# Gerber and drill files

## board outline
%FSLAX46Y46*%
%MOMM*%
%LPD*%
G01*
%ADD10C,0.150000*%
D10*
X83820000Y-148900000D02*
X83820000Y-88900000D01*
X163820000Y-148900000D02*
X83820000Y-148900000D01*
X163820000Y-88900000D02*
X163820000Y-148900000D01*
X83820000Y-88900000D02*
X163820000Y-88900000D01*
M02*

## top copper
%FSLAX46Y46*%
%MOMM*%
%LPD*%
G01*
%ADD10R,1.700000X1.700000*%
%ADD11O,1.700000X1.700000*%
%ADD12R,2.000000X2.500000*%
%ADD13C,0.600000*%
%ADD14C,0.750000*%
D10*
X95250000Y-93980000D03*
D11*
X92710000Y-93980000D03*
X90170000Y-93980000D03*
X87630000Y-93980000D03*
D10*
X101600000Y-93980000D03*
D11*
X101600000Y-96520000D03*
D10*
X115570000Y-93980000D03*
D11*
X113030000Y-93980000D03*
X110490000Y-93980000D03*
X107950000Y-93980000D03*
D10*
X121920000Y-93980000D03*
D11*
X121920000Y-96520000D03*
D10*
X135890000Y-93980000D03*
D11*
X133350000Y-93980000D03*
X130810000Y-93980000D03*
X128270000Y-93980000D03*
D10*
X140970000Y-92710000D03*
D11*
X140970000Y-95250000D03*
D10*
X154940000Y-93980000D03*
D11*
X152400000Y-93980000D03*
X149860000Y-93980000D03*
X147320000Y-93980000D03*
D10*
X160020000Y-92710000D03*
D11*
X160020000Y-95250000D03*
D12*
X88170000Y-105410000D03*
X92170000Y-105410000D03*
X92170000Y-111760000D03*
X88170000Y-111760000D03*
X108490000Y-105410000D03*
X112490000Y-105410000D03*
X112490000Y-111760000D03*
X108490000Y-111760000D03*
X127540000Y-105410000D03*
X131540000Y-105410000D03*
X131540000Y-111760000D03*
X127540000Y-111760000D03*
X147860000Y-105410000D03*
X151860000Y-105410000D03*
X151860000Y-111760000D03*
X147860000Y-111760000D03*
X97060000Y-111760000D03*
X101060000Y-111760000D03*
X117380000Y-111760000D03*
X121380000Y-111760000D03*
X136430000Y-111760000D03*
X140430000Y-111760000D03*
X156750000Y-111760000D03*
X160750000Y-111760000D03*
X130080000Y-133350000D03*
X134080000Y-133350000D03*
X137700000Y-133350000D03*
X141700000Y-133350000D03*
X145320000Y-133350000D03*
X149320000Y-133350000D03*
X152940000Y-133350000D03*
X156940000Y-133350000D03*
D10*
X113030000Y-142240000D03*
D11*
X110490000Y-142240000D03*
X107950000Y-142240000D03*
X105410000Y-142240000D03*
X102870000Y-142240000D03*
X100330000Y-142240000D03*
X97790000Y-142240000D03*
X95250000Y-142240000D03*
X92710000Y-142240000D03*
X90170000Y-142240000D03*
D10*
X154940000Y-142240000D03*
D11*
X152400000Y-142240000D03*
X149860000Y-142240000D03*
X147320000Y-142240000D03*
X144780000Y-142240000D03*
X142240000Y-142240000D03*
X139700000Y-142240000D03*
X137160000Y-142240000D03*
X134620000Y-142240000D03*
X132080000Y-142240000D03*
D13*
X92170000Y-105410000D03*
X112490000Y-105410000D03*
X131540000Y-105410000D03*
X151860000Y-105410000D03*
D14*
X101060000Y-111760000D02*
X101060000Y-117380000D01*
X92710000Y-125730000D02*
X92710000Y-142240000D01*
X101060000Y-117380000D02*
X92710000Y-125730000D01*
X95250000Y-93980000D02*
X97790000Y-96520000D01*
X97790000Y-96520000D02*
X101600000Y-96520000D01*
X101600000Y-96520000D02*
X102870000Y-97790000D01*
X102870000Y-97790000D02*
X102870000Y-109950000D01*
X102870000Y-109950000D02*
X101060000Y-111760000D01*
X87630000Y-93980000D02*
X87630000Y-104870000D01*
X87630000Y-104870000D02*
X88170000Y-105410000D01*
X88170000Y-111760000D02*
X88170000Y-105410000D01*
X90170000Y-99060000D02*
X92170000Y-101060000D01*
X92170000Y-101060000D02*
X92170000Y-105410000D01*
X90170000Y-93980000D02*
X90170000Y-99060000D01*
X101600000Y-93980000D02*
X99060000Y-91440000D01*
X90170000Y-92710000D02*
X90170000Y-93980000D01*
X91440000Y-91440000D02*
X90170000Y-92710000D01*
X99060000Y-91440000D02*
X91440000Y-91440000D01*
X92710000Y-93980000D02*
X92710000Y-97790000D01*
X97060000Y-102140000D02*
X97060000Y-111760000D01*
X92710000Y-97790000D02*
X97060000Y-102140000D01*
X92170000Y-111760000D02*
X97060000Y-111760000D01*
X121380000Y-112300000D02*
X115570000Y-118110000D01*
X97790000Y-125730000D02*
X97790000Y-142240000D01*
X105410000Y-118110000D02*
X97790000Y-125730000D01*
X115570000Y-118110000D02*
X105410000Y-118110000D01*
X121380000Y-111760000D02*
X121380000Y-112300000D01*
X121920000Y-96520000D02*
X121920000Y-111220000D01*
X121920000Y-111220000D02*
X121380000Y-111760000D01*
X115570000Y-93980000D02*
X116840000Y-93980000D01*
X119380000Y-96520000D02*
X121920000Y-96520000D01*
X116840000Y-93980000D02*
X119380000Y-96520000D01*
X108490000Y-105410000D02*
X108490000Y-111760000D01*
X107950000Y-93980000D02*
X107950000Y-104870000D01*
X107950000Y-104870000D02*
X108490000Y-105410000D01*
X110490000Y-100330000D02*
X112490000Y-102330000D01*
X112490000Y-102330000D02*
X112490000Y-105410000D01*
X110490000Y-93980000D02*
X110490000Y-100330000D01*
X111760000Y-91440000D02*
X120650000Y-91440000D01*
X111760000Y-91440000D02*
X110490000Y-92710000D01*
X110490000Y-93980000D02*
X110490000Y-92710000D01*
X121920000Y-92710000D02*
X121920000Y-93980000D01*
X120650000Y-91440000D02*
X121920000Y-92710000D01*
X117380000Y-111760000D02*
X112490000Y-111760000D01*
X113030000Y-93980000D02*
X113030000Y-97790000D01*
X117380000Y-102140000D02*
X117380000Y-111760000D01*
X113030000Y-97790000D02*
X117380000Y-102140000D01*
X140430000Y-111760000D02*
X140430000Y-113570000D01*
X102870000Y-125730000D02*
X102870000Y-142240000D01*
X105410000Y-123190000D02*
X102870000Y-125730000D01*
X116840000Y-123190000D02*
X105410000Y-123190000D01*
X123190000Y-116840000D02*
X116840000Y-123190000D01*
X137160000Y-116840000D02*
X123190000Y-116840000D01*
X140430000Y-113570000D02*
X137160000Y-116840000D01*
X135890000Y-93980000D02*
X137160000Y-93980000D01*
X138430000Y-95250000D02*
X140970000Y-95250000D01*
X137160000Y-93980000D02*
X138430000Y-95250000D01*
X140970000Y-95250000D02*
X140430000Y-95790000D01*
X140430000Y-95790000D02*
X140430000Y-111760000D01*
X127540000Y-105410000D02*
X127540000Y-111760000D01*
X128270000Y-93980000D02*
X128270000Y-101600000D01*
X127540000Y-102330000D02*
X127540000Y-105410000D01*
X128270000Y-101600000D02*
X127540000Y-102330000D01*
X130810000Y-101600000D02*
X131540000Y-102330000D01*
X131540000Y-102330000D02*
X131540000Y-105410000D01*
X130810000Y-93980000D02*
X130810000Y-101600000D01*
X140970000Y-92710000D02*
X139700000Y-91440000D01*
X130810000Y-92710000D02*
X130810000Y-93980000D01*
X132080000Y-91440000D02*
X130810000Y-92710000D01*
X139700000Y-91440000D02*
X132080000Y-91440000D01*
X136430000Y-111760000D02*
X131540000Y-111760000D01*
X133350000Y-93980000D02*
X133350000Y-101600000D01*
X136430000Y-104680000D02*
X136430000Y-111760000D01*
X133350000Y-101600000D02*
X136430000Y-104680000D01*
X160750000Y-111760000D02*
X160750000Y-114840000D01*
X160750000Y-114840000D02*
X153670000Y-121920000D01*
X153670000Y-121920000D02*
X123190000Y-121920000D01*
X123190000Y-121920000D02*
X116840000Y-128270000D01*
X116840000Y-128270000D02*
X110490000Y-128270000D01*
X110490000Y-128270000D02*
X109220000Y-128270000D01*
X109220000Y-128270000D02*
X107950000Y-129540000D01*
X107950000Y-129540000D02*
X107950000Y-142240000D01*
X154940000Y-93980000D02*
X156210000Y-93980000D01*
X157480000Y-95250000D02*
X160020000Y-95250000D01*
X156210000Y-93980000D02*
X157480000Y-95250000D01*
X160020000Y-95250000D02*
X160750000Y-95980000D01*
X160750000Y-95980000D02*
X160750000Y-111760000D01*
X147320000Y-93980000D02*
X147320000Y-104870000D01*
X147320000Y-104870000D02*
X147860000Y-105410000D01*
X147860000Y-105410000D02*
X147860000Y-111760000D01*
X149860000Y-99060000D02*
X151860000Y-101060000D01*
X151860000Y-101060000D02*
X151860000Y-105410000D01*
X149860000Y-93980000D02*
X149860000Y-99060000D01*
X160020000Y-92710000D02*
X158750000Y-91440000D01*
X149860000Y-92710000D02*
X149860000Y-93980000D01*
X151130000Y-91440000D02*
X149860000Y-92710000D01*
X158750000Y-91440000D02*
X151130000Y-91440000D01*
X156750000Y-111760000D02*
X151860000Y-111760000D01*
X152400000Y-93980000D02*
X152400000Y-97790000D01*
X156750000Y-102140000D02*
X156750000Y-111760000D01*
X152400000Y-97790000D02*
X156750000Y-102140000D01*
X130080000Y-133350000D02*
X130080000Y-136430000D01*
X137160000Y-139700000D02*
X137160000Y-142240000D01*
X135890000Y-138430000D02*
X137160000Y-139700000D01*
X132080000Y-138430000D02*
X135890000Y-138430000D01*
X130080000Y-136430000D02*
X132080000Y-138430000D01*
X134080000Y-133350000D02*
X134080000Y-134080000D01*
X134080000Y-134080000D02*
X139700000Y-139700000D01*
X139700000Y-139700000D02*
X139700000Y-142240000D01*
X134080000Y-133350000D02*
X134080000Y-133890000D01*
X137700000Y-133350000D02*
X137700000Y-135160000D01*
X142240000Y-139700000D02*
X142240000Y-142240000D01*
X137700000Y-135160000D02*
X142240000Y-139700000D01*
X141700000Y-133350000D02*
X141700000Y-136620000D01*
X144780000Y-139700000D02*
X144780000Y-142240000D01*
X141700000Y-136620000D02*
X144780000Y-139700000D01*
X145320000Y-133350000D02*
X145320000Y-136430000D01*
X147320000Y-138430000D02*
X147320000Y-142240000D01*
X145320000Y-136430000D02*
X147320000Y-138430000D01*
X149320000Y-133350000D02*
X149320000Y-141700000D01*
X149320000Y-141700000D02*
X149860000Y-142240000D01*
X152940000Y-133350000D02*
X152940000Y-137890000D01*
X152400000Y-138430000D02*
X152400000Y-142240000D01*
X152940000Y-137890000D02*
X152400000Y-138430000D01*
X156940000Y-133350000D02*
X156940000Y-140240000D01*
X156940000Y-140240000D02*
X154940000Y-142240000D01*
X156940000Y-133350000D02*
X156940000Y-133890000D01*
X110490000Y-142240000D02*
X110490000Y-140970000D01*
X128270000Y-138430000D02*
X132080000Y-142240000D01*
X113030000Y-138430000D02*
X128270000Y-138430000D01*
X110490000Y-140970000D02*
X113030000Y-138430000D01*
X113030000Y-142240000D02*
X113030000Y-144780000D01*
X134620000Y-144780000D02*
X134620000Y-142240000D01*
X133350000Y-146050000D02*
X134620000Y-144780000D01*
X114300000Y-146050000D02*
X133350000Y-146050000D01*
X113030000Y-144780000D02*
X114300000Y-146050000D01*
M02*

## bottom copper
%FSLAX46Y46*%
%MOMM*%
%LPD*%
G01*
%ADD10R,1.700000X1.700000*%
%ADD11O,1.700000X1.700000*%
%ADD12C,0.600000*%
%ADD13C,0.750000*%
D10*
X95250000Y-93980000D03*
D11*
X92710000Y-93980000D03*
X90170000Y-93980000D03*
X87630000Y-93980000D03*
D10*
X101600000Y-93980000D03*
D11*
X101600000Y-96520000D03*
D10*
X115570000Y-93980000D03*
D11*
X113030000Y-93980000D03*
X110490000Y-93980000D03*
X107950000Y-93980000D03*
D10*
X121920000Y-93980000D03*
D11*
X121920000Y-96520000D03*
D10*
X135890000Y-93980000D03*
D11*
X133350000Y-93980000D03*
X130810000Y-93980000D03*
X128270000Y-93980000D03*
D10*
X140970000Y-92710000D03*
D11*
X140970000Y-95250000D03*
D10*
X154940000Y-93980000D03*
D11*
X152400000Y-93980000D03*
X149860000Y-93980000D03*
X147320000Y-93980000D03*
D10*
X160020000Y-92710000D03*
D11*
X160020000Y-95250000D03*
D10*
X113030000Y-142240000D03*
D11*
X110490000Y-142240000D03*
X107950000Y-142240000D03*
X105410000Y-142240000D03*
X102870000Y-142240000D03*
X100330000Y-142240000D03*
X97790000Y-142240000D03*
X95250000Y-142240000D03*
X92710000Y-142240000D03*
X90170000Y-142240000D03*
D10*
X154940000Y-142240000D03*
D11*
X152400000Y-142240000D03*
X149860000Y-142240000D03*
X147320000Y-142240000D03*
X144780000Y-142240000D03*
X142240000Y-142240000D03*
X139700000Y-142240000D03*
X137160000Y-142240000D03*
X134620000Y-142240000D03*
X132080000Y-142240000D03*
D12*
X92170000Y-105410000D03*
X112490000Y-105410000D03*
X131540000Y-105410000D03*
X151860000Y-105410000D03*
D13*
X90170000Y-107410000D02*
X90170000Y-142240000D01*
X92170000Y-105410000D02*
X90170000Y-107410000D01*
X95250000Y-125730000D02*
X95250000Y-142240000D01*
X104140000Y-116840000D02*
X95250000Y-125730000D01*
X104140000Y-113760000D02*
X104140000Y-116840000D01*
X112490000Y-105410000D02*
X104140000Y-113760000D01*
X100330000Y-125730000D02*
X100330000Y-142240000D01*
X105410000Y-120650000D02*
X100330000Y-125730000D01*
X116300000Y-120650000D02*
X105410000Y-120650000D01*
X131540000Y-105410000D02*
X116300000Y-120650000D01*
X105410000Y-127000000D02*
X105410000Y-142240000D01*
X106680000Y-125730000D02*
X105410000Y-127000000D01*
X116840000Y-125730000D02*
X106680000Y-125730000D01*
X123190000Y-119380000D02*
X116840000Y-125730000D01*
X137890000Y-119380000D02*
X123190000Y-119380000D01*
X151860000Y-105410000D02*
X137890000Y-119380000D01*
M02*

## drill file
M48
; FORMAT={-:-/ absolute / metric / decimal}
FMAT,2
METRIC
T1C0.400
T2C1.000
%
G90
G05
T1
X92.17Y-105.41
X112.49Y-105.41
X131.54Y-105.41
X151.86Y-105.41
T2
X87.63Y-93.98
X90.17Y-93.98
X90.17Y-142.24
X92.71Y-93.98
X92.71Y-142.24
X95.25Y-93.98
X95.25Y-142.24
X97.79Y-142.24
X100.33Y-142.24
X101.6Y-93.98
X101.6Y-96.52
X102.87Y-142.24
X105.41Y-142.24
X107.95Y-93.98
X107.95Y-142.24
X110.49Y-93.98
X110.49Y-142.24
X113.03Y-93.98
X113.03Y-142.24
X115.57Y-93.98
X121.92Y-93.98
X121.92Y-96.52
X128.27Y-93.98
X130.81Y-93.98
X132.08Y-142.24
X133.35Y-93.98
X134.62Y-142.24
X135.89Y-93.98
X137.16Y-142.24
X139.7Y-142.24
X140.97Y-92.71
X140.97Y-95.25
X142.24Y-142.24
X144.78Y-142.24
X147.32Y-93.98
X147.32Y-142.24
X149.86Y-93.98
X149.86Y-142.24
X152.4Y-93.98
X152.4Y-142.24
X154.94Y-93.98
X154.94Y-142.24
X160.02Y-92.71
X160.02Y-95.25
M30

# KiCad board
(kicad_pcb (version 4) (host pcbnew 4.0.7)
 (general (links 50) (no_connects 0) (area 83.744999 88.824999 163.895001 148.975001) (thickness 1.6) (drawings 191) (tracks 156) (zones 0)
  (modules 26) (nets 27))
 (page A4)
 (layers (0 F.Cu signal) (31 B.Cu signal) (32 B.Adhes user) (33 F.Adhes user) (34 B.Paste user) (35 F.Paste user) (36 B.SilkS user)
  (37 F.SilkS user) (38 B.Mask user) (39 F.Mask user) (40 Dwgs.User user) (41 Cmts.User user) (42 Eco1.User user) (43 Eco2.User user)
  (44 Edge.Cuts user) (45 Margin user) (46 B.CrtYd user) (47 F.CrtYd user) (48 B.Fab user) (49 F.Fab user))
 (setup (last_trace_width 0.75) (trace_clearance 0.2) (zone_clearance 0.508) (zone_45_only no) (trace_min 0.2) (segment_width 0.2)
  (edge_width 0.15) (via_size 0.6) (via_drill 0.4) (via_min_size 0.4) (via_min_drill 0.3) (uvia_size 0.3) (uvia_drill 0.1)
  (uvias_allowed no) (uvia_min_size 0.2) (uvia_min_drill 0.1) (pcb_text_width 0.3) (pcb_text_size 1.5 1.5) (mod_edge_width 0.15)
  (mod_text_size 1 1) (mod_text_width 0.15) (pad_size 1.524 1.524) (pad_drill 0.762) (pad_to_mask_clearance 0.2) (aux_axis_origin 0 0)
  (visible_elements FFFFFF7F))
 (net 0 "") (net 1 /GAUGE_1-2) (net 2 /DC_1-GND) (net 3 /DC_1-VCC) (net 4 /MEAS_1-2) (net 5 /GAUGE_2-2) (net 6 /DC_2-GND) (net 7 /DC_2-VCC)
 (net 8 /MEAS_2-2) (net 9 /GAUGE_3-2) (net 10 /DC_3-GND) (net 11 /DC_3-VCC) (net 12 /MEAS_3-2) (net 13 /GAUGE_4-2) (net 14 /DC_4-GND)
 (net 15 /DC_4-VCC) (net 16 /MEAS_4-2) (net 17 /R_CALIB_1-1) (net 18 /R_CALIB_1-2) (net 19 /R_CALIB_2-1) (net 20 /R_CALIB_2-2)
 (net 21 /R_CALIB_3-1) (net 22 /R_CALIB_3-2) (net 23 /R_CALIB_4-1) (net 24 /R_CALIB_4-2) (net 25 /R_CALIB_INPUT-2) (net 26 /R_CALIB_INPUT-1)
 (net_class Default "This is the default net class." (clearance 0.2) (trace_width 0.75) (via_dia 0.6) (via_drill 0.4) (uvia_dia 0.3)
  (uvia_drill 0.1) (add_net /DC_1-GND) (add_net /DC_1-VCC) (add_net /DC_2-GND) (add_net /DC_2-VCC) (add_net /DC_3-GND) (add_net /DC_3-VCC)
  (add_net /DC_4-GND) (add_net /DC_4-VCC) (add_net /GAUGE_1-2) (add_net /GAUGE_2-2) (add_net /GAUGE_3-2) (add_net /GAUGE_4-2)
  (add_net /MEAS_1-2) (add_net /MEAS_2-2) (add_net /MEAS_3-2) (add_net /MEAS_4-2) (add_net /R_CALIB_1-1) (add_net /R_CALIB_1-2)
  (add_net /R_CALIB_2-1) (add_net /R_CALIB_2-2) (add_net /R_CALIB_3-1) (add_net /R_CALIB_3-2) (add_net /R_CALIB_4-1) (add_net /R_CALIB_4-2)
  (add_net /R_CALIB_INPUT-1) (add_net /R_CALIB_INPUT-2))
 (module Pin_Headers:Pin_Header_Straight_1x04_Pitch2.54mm (layer F.Cu) (at 95.25 93.98 270)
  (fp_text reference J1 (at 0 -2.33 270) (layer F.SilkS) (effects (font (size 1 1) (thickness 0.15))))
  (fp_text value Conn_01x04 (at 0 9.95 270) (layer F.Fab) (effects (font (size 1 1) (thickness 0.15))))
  (pad 1 thru_hole rect (at 0 0 270) (size 1.7 1.7) (drill 1) (layers *.Cu *.Mask) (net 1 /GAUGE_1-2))
  (pad 2 thru_hole oval (at 0 2.54 270) (size 1.7 1.7) (drill 1) (layers *.Cu *.Mask) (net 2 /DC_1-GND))
  (pad 3 thru_hole oval (at 0 5.08 270) (size 1.7 1.7) (drill 1) (layers *.Cu *.Mask) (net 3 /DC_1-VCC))
  (pad 4 thru_hole oval (at 0 7.62 270) (size 1.7 1.7) (drill 1) (layers *.Cu *.Mask) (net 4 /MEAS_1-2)))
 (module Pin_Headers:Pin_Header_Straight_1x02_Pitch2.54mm (layer F.Cu) (at 101.6 93.98)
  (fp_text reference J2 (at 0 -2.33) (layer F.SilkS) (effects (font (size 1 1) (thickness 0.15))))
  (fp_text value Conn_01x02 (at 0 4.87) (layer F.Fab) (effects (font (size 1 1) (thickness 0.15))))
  (pad 1 thru_hole rect (at 0 0) (size 1.7 1.7) (drill 1) (layers *.Cu *.Mask) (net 3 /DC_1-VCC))
  (pad 2 thru_hole oval (at 0 2.54) (size 1.7 1.7) (drill 1) (layers *.Cu *.Mask) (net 1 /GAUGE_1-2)))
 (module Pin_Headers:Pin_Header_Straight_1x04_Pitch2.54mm (layer F.Cu) (at 115.57 93.98 270)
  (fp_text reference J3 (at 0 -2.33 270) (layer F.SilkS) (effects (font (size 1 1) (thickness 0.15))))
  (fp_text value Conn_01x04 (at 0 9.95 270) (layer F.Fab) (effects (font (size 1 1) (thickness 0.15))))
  (pad 1 thru_hole rect (at 0 0 270) (size 1.7 1.7) (drill 1) (layers *.Cu *.Mask) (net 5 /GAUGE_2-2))
  (pad 2 thru_hole oval (at 0 2.54 270) (size 1.7 1.7) (drill 1) (layers *.Cu *.Mask) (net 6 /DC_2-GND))
  (pad 3 thru_hole oval (at 0 5.08 270) (size 1.7 1.7) (drill 1) (layers *.Cu *.Mask) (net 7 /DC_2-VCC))
  (pad 4 thru_hole oval (at 0 7.62 270) (size 1.7 1.7) (drill 1) (layers *.Cu *.Mask) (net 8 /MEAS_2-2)))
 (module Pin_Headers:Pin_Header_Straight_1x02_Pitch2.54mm (layer F.Cu) (at 121.92 93.98)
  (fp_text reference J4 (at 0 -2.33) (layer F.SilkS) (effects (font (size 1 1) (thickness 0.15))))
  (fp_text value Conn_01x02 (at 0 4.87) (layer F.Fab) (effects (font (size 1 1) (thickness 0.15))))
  (pad 1 thru_hole rect (at 0 0) (size 1.7 1.7) (drill 1) (layers *.Cu *.Mask) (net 7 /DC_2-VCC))
  (pad 2 thru_hole oval (at 0 2.54) (size 1.7 1.7) (drill 1) (layers *.Cu *.Mask) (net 5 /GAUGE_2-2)))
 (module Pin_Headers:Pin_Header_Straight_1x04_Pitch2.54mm (layer F.Cu) (at 135.89 93.98 270)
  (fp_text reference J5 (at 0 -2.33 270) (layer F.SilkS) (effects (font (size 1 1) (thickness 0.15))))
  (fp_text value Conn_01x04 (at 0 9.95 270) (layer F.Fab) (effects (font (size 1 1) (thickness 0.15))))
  (pad 1 thru_hole rect (at 0 0 270) (size 1.7 1.7) (drill 1) (layers *.Cu *.Mask) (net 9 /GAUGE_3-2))
  (pad 2 thru_hole oval (at 0 2.54 270) (size 1.7 1.7) (drill 1) (layers *.Cu *.Mask) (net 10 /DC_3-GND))
  (pad 3 thru_hole oval (at 0 5.08 270) (size 1.7 1.7) (drill 1) (layers *.Cu *.Mask) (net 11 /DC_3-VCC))
  (pad 4 thru_hole oval (at 0 7.62 270) (size 1.7 1.7) (drill 1) (layers *.Cu *.Mask) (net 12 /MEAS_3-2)))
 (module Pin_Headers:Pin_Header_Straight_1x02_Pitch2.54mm (layer F.Cu) (at 140.97 92.71)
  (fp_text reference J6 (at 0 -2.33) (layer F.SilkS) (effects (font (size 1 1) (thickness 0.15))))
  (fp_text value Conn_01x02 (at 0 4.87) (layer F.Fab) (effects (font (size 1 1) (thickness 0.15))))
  (pad 1 thru_hole rect (at 0 0) (size 1.7 1.7) (drill 1) (layers *.Cu *.Mask) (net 11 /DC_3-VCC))
  (pad 2 thru_hole oval (at 0 2.54) (size 1.7 1.7) (drill 1) (layers *.Cu *.Mask) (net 9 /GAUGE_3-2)))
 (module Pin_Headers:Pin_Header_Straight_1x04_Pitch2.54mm (layer F.Cu) (at 154.94 93.98 270)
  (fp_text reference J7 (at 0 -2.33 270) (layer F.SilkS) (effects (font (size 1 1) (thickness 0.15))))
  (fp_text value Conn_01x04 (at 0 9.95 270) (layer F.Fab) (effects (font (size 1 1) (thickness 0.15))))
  (pad 1 thru_hole rect (at 0 0 270) (size 1.7 1.7) (drill 1) (layers *.Cu *.Mask) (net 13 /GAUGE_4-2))
  (pad 2 thru_hole oval (at 0 2.54 270) (size 1.7 1.7) (drill 1) (layers *.Cu *.Mask) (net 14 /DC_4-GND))
  (pad 3 thru_hole oval (at 0 5.08 270) (size 1.7 1.7) (drill 1) (layers *.Cu *.Mask) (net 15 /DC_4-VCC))
  (pad 4 thru_hole oval (at 0 7.62 270) (size 1.7 1.7) (drill 1) (layers *.Cu *.Mask) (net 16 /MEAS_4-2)))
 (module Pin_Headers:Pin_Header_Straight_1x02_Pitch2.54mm (layer F.Cu) (at 160.02 92.71)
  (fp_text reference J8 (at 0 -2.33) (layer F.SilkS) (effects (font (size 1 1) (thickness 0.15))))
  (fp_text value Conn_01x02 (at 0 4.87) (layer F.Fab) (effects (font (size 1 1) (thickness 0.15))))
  (pad 1 thru_hole rect (at 0 0) (size 1.7 1.7) (drill 1) (layers *.Cu *.Mask) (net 15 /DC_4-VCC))
  (pad 2 thru_hole oval (at 0 2.54) (size 1.7 1.7) (drill 1) (layers *.Cu *.Mask) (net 13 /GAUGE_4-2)))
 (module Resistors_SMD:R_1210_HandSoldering (layer F.Cu) (at 90.17 105.41)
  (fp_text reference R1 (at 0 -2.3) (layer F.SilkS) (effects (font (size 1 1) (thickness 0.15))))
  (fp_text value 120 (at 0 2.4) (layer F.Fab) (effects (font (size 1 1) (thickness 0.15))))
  (pad 1 smd rect (at -2 0) (size 2 2.5) (layers F.Cu F.Paste F.Mask) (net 4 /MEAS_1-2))
  (pad 2 smd rect (at 2 0) (size 2 2.5) (layers F.Cu F.Paste F.Mask) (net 3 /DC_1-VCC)))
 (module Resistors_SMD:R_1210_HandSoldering (layer F.Cu) (at 90.17 111.76 180)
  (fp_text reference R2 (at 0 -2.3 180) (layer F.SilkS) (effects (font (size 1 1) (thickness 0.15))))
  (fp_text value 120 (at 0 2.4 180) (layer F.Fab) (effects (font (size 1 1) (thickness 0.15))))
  (pad 1 smd rect (at -2 0 180) (size 2 2.5) (layers F.Cu F.Paste F.Mask) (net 2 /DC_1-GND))
  (pad 2 smd rect (at 2 0 180) (size 2 2.5) (layers F.Cu F.Paste F.Mask) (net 4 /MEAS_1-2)))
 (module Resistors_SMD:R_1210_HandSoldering (layer F.Cu) (at 110.49 105.41)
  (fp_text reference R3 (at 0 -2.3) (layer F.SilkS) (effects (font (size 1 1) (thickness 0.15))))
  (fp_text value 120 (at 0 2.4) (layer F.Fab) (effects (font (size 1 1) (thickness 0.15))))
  (pad 1 smd rect (at -2 0) (size 2 2.5) (layers F.Cu F.Paste F.Mask) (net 8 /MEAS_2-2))
  (pad 2 smd rect (at 2 0) (size 2 2.5) (layers F.Cu F.Paste F.Mask) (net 7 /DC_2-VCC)))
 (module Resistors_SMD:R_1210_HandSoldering (layer F.Cu) (at 110.49 111.76 180)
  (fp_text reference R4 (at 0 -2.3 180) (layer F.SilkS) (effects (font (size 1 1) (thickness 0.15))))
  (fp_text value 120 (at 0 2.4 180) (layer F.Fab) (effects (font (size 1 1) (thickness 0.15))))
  (pad 1 smd rect (at -2 0 180) (size 2 2.5) (layers F.Cu F.Paste F.Mask) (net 6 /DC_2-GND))
  (pad 2 smd rect (at 2 0 180) (size 2 2.5) (layers F.Cu F.Paste F.Mask) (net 8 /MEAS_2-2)))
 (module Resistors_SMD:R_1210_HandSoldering (layer F.Cu) (at 129.54 105.41)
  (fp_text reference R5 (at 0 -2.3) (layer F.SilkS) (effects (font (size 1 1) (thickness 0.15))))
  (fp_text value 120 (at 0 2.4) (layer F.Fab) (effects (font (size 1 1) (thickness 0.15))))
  (pad 1 smd rect (at -2 0) (size 2 2.5) (layers F.Cu F.Paste F.Mask) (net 12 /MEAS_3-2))
  (pad 2 smd rect (at 2 0) (size 2 2.5) (layers F.Cu F.Paste F.Mask) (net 11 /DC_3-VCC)))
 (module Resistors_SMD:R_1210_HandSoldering (layer F.Cu) (at 129.54 111.76 180)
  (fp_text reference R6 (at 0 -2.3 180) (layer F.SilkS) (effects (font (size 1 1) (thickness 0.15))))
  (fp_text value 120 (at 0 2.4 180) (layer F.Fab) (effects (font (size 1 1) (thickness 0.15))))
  (pad 1 smd rect (at -2 0 180) (size 2 2.5) (layers F.Cu F.Paste F.Mask) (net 10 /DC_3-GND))
  (pad 2 smd rect (at 2 0 180) (size 2 2.5) (layers F.Cu F.Paste F.Mask) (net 12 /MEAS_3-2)))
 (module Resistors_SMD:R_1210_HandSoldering (layer F.Cu) (at 149.86 105.41)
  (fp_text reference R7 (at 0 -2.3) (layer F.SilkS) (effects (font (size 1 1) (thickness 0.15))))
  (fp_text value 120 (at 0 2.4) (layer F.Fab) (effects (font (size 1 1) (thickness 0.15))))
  (pad 1 smd rect (at -2 0) (size 2 2.5) (layers F.Cu F.Paste F.Mask) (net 16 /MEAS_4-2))
  (pad 2 smd rect (at 2 0) (size 2 2.5) (layers F.Cu F.Paste F.Mask) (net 15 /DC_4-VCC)))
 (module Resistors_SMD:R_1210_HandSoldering (layer F.Cu) (at 149.86 111.76 180)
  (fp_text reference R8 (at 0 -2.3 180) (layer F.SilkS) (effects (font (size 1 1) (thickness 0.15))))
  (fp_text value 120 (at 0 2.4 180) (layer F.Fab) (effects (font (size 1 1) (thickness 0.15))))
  (pad 1 smd rect (at -2 0 180) (size 2 2.5) (layers F.Cu F.Paste F.Mask) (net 14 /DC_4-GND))
  (pad 2 smd rect (at 2 0 180) (size 2 2.5) (layers F.Cu F.Paste F.Mask) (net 16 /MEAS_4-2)))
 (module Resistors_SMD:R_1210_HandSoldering (layer F.Cu) (at 99.06 111.76)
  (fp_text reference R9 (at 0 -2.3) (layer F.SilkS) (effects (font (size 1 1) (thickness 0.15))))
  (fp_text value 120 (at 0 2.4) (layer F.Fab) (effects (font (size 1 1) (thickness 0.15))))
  (pad 1 smd rect (at -2 0) (size 2 2.5) (layers F.Cu F.Paste F.Mask) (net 2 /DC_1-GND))
  (pad 2 smd rect (at 2 0) (size 2 2.5) (layers F.Cu F.Paste F.Mask) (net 1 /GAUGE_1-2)))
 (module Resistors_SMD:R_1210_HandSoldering (layer F.Cu) (at 119.38 111.76)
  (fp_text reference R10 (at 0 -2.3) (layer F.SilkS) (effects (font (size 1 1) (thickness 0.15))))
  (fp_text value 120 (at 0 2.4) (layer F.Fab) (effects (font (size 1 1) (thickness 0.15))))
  (pad 1 smd rect (at -2 0) (size 2 2.5) (layers F.Cu F.Paste F.Mask) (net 6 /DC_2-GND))
  (pad 2 smd rect (at 2 0) (size 2 2.5) (layers F.Cu F.Paste F.Mask) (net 5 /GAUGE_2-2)))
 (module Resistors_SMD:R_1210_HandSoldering (layer F.Cu) (at 138.43 111.76)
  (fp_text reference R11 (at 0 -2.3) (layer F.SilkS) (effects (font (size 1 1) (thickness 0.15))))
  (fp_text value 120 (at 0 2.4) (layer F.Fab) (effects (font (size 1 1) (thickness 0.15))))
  (pad 1 smd rect (at -2 0) (size 2 2.5) (layers F.Cu F.Paste F.Mask) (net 10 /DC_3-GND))
  (pad 2 smd rect (at 2 0) (size 2 2.5) (layers F.Cu F.Paste F.Mask) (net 9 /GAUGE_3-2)))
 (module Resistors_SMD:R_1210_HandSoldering (layer F.Cu) (at 158.75 111.76)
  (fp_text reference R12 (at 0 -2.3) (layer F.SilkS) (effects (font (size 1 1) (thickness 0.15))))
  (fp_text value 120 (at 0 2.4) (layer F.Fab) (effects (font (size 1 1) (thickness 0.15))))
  (pad 1 smd rect (at -2 0) (size 2 2.5) (layers F.Cu F.Paste F.Mask) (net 14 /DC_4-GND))
  (pad 2 smd rect (at 2 0) (size 2 2.5) (layers F.Cu F.Paste F.Mask) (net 13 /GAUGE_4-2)))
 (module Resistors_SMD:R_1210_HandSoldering (layer F.Cu) (at 132.08 133.35)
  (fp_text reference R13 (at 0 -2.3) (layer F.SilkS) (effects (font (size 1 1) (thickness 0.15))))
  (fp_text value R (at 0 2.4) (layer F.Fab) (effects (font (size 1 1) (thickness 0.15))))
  (pad 1 smd rect (at -2 0) (size 2 2.5) (layers F.Cu F.Paste F.Mask) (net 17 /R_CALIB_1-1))
  (pad 2 smd rect (at 2 0) (size 2 2.5) (layers F.Cu F.Paste F.Mask) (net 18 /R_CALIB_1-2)))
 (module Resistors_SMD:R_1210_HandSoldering (layer F.Cu) (at 139.7 133.35)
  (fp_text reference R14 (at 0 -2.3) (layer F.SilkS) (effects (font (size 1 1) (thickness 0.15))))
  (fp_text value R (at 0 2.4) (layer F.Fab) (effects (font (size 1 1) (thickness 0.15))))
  (pad 1 smd rect (at -2 0) (size 2 2.5) (layers F.Cu F.Paste F.Mask) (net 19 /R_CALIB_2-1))
  (pad 2 smd rect (at 2 0) (size 2 2.5) (layers F.Cu F.Paste F.Mask) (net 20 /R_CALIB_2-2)))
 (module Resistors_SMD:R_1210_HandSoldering (layer F.Cu) (at 147.32 133.35)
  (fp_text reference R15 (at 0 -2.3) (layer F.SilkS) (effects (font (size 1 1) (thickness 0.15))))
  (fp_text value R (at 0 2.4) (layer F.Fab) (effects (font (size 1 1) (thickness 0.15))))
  (pad 1 smd rect (at -2 0) (size 2 2.5) (layers F.Cu F.Paste F.Mask) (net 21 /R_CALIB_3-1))
  (pad 2 smd rect (at 2 0) (size 2 2.5) (layers F.Cu F.Paste F.Mask) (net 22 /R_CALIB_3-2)))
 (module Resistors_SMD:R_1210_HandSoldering (layer F.Cu) (at 154.94 133.35)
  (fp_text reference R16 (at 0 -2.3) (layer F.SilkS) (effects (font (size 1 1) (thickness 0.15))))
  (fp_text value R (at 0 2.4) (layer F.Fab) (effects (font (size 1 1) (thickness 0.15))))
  (pad 1 smd rect (at -2 0) (size 2 2.5) (layers F.Cu F.Paste F.Mask) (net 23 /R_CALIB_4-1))
  (pad 2 smd rect (at 2 0) (size 2 2.5) (layers F.Cu F.Paste F.Mask) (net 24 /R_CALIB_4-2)))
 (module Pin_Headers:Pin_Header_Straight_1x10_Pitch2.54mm (layer F.Cu) (at 113.03 142.24 270)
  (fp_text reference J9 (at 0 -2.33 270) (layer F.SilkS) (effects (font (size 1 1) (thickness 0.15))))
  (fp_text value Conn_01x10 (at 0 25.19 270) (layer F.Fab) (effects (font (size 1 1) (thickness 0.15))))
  (pad 1 thru_hole rect (at 0 0 270) (size 1.7 1.7) (drill 1) (layers *.Cu *.Mask) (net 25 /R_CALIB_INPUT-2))
  (pad 2 thru_hole oval (at 0 2.54 270) (size 1.7 1.7) (drill 1) (layers *.Cu *.Mask) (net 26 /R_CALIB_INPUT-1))
  (pad 3 thru_hole oval (at 0 5.08 270) (size 1.7 1.7) (drill 1) (layers *.Cu *.Mask) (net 13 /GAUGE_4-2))
  (pad 4 thru_hole oval (at 0 7.62 270) (size 1.7 1.7) (drill 1) (layers *.Cu *.Mask) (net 15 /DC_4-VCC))
  (pad 5 thru_hole oval (at 0 10.16 270) (size 1.7 1.7) (drill 1) (layers *.Cu *.Mask) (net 9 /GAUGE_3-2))
  (pad 6 thru_hole oval (at 0 12.7 270) (size 1.7 1.7) (drill 1) (layers *.Cu *.Mask) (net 11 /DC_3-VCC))
  (pad 7 thru_hole oval (at 0 15.24 270) (size 1.7 1.7) (drill 1) (layers *.Cu *.Mask) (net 5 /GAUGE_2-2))
  (pad 8 thru_hole oval (at 0 17.78 270) (size 1.7 1.7) (drill 1) (layers *.Cu *.Mask) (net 7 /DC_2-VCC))
  (pad 9 thru_hole oval (at 0 20.32 270) (size 1.7 1.7) (drill 1) (layers *.Cu *.Mask) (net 1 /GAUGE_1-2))
  (pad 10 thru_hole oval (at 0 22.86 270) (size 1.7 1.7) (drill 1) (layers *.Cu *.Mask) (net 3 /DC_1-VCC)))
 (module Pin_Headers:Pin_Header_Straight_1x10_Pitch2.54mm (layer F.Cu) (at 154.94 142.24 270)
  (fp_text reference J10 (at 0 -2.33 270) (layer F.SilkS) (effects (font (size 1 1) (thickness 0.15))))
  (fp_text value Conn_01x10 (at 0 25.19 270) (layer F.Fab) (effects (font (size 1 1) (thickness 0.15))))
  (pad 1 thru_hole rect (at 0 0 270) (size 1.7 1.7) (drill 1) (layers *.Cu *.Mask) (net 24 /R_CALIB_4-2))
  (pad 2 thru_hole oval (at 0 2.54 270) (size 1.7 1.7) (drill 1) (layers *.Cu *.Mask) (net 23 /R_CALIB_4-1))
  (pad 3 thru_hole oval (at 0 5.08 270) (size 1.7 1.7) (drill 1) (layers *.Cu *.Mask) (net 22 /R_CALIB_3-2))
  (pad 4 thru_hole oval (at 0 7.62 270) (size 1.7 1.7) (drill 1) (layers *.Cu *.Mask) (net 21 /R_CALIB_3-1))
  (pad 5 thru_hole oval (at 0 10.16 270) (size 1.7 1.7) (drill 1) (layers *.Cu *.Mask) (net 20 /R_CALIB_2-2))
  (pad 6 thru_hole oval (at 0 12.7 270) (size 1.7 1.7) (drill 1) (layers *.Cu *.Mask) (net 19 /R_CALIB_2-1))
  (pad 7 thru_hole oval (at 0 15.24 270) (size 1.7 1.7) (drill 1) (layers *.Cu *.Mask) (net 18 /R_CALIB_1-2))
  (pad 8 thru_hole oval (at 0 17.78 270) (size 1.7 1.7) (drill 1) (layers *.Cu *.Mask) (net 17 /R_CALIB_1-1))
  (pad 9 thru_hole oval (at 0 20.32 270) (size 1.7 1.7) (drill 1) (layers *.Cu *.Mask) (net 25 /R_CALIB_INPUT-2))
  (pad 10 thru_hole oval (at 0 22.86 270) (size 1.7 1.7) (drill 1) (layers *.Cu *.Mask) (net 26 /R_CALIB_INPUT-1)))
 (gr_line (start 83.82 148.9) (end 83.82 88.9) (angle 90) (layer Edge.Cuts) (width 0.15))
 (gr_line (start 163.82 148.9) (end 83.82 148.9) (angle 90) (layer Edge.Cuts) (width 0.15))
 (gr_line (start 163.82 88.9) (end 163.82 148.9) (angle 90) (layer Edge.Cuts) (width 0.15))
 (gr_line (start 83.82 88.9) (end 163.82 88.9) (angle 90) (layer Edge.Cuts) (width 0.15))
 (segment (start 101.06 111.76) (end 101.06 117.38) (width 0.75) (layer F.Cu) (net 1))
 (segment (start 92.71 125.73) (end 92.71 142.24) (width 0.75) (layer F.Cu) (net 1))
 (segment (start 101.06 117.38) (end 92.71 125.73) (width 0.75) (layer F.Cu) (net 1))
 (segment (start 95.25 93.98) (end 97.79 96.52) (width 0.75) (layer F.Cu) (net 1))
 (segment (start 97.79 96.52) (end 101.6 96.52) (width 0.75) (layer F.Cu) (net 1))
 (segment (start 101.6 96.52) (end 102.87 97.79) (width 0.75) (layer F.Cu) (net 1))
 (segment (start 102.87 97.79) (end 102.87 109.95) (width 0.75) (layer F.Cu) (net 1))
 (segment (start 102.87 109.95) (end 101.06 111.76) (width 0.75) (layer F.Cu) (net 1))
 (segment (start 87.63 93.98) (end 87.63 104.87) (width 0.75) (layer F.Cu) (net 4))
 (segment (start 87.63 104.87) (end 88.17 105.41) (width 0.75) (layer F.Cu) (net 4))
 (segment (start 88.17 111.76) (end 88.17 105.41) (width 0.75) (layer F.Cu) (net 4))
 (via (at 92.17 105.41) (size 0.6) (drill 0.4) (layers F.Cu B.Cu) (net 3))
 (segment (start 90.17 99.06) (end 92.17 101.06) (width 0.75) (layer F.Cu) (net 3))
 (segment (start 92.17 101.06) (end 92.17 105.41) (width 0.75) (layer F.Cu) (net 3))
 (segment (start 90.17 93.98) (end 90.17 99.06) (width 0.75) (layer F.Cu) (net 3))
 (segment (start 90.17 107.41) (end 90.17 142.24) (width 0.75) (layer B.Cu) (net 3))
 (segment (start 92.17 105.41) (end 90.17 107.41) (width 0.75) (layer B.Cu) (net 3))
 (segment (start 101.6 93.98) (end 99.06 91.44) (width 0.75) (layer F.Cu) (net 3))
 (segment (start 90.17 92.71) (end 90.17 93.98) (width 0.75) (layer F.Cu) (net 3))
 (segment (start 91.44 91.44) (end 90.17 92.71) (width 0.75) (layer F.Cu) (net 3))
 (segment (start 99.06 91.44) (end 91.44 91.44) (width 0.75) (layer F.Cu) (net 3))
 (segment (start 92.71 93.98) (end 92.71 97.79) (width 0.75) (layer F.Cu) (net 2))
 (segment (start 97.06 102.14) (end 97.06 111.76) (width 0.75) (layer F.Cu) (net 2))
 (segment (start 92.71 97.79) (end 97.06 102.14) (width 0.75) (layer F.Cu) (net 2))
 (segment (start 92.17 111.76) (end 97.06 111.76) (width 0.75) (layer F.Cu) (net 2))
 (segment (start 121.38 112.3) (end 115.57 118.11) (width 0.75) (layer F.Cu) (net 5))
 (segment (start 97.79 125.73) (end 97.79 142.24) (width 0.75) (layer F.Cu) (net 5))
 (segment (start 105.41 118.11) (end 97.79 125.73) (width 0.75) (layer F.Cu) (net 5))
 (segment (start 115.57 118.11) (end 105.41 118.11) (width 0.75) (layer F.Cu) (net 5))
 (segment (start 121.38 111.76) (end 121.38 112.3) (width 0.75) (layer F.Cu) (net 5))
 (segment (start 121.92 96.52) (end 121.92 111.22) (width 0.75) (layer F.Cu) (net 5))
 (segment (start 121.92 111.22) (end 121.38 111.76) (width 0.75) (layer F.Cu) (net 5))
 (segment (start 115.57 93.98) (end 116.84 93.98) (width 0.75) (layer F.Cu) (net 5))
 (segment (start 119.38 96.52) (end 121.92 96.52) (width 0.75) (layer F.Cu) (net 5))
 (segment (start 116.84 93.98) (end 119.38 96.52) (width 0.75) (layer F.Cu) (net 5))
 (segment (start 108.49 105.41) (end 108.49 111.76) (width 0.75) (layer F.Cu) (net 8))
 (segment (start 107.95 93.98) (end 107.95 104.87) (width 0.75) (layer F.Cu) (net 8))
 (segment (start 107.95 104.87) (end 108.49 105.41) (width 0.75) (layer F.Cu) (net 8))
 (via (at 112.49 105.41) (size 0.6) (drill 0.4) (layers F.Cu B.Cu) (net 7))
 (segment (start 110.49 100.33) (end 112.49 102.33) (width 0.75) (layer F.Cu) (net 7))
 (segment (start 112.49 102.33) (end 112.49 105.41) (width 0.75) (layer F.Cu) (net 7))
 (segment (start 110.49 93.98) (end 110.49 100.33) (width 0.75) (layer F.Cu) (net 7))
 (segment (start 95.25 125.73) (end 95.25 142.24) (width 0.75) (layer B.Cu) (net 7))
 (segment (start 104.14 116.84) (end 95.25 125.73) (width 0.75) (layer B.Cu) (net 7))
 (segment (start 104.14 113.76) (end 104.14 116.84) (width 0.75) (layer B.Cu) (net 7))
 (segment (start 112.49 105.41) (end 104.14 113.76) (width 0.75) (layer B.Cu) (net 7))
 (segment (start 111.76 91.44) (end 120.65 91.44) (width 0.75) (layer F.Cu) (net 7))
 (segment (start 111.76 91.44) (end 110.49 92.71) (width 0.75) (layer F.Cu) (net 7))
 (segment (start 110.49 93.98) (end 110.49 92.71) (width 0.75) (layer F.Cu) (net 7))
 (segment (start 121.92 92.71) (end 121.92 93.98) (width 0.75) (layer F.Cu) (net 7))
 (segment (start 120.65 91.44) (end 121.92 92.71) (width 0.75) (layer F.Cu) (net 7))
 (segment (start 117.38 111.76) (end 112.49 111.76) (width 0.75) (layer F.Cu) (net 6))
 (segment (start 113.03 93.98) (end 113.03 97.79) (width 0.75) (layer F.Cu) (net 6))
 (segment (start 117.38 102.14) (end 117.38 111.76) (width 0.75) (layer F.Cu) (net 6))
 (segment (start 113.03 97.79) (end 117.38 102.14) (width 0.75) (layer F.Cu) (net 6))
 (segment (start 140.43 111.76) (end 140.43 113.57) (width 0.75) (layer F.Cu) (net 9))
 (segment (start 102.87 125.73) (end 102.87 142.24) (width 0.75) (layer F.Cu) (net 9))
 (segment (start 105.41 123.19) (end 102.87 125.73) (width 0.75) (layer F.Cu) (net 9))
 (segment (start 116.84 123.19) (end 105.41 123.19) (width 0.75) (layer F.Cu) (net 9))
 (segment (start 123.19 116.84) (end 116.84 123.19) (width 0.75) (layer F.Cu) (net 9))
 (segment (start 137.16 116.84) (end 123.19 116.84) (width 0.75) (layer F.Cu) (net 9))
 (segment (start 140.43 113.57) (end 137.16 116.84) (width 0.75) (layer F.Cu) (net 9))
 (segment (start 135.89 93.98) (end 137.16 93.98) (width 0.75) (layer F.Cu) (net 9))
 (segment (start 138.43 95.25) (end 140.97 95.25) (width 0.75) (layer F.Cu) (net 9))
 (segment (start 137.16 93.98) (end 138.43 95.25) (width 0.75) (layer F.Cu) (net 9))
 (segment (start 140.97 95.25) (end 140.43 95.79) (width 0.75) (layer F.Cu) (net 9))
 (segment (start 140.43 95.79) (end 140.43 111.76) (width 0.75) (layer F.Cu) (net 9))
 (segment (start 127.54 105.41) (end 127.54 111.76) (width 0.75) (layer F.Cu) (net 12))
 (segment (start 128.27 93.98) (end 128.27 101.6) (width 0.75) (layer F.Cu) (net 12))
 (segment (start 127.54 102.33) (end 127.54 105.41) (width 0.75) (layer F.Cu) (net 12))
 (segment (start 128.27 101.6) (end 127.54 102.33) (width 0.75) (layer F.Cu) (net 12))
 (via (at 131.54 105.41) (size 0.6) (drill 0.4) (layers F.Cu B.Cu) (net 11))
 (segment (start 130.81 101.6) (end 131.54 102.33) (width 0.75) (layer F.Cu) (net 11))
 (segment (start 131.54 102.33) (end 131.54 105.41) (width 0.75) (layer F.Cu) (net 11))
 (segment (start 130.81 93.98) (end 130.81 101.6) (width 0.75) (layer F.Cu) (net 11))
 (segment (start 100.33 125.73) (end 100.33 142.24) (width 0.75) (layer B.Cu) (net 11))
 (segment (start 105.41 120.65) (end 100.33 125.73) (width 0.75) (layer B.Cu) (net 11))
 (segment (start 116.3 120.65) (end 105.41 120.65) (width 0.75) (layer B.Cu) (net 11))
 (segment (start 131.54 105.41) (end 116.3 120.65) (width 0.75) (layer B.Cu) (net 11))
 (segment (start 140.97 92.71) (end 139.7 91.44) (width 0.75) (layer F.Cu) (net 11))
 (segment (start 130.81 92.71) (end 130.81 93.98) (width 0.75) (layer F.Cu) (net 11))
 (segment (start 132.08 91.44) (end 130.81 92.71) (width 0.75) (layer F.Cu) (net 11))
 (segment (start 139.7 91.44) (end 132.08 91.44) (width 0.75) (layer F.Cu) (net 11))
 (segment (start 136.43 111.76) (end 131.54 111.76) (width 0.75) (layer F.Cu) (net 10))
 (segment (start 133.35 93.98) (end 133.35 101.6) (width 0.75) (layer F.Cu) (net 10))
 (segment (start 136.43 104.68) (end 136.43 111.76) (width 0.75) (layer F.Cu) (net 10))
 (segment (start 133.35 101.6) (end 136.43 104.68) (width 0.75) (layer F.Cu) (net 10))
 (segment (start 160.75 111.76) (end 160.75 114.84) (width 0.75) (layer F.Cu) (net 13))
 (segment (start 160.75 114.84) (end 153.67 121.92) (width 0.75) (layer F.Cu) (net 13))
 (segment (start 153.67 121.92) (end 123.19 121.92) (width 0.75) (layer F.Cu) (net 13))
 (segment (start 123.19 121.92) (end 116.84 128.27) (width 0.75) (layer F.Cu) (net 13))
 (segment (start 116.84 128.27) (end 110.49 128.27) (width 0.75) (layer F.Cu) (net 13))
 (segment (start 110.49 128.27) (end 109.22 128.27) (width 0.75) (layer F.Cu) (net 13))
 (segment (start 109.22 128.27) (end 107.95 129.54) (width 0.75) (layer F.Cu) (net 13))
 (segment (start 107.95 129.54) (end 107.95 142.24) (width 0.75) (layer F.Cu) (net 13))
 (segment (start 154.94 93.98) (end 156.21 93.98) (width 0.75) (layer F.Cu) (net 13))
 (segment (start 157.48 95.25) (end 160.02 95.25) (width 0.75) (layer F.Cu) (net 13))
 (segment (start 156.21 93.98) (end 157.48 95.25) (width 0.75) (layer F.Cu) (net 13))
 (segment (start 160.02 95.25) (end 160.75 95.98) (width 0.75) (layer F.Cu) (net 13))
 (segment (start 160.75 95.98) (end 160.75 111.76) (width 0.75) (layer F.Cu) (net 13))
 (segment (start 147.32 93.98) (end 147.32 104.87) (width 0.75) (layer F.Cu) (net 16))
 (segment (start 147.32 104.87) (end 147.86 105.41) (width 0.75) (layer F.Cu) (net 16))
 (segment (start 147.86 105.41) (end 147.86 111.76) (width 0.75) (layer F.Cu) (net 16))
 (via (at 151.86 105.41) (size 0.6) (drill 0.4) (layers F.Cu B.Cu) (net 15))
 (segment (start 149.86 99.06) (end 151.86 101.06) (width 0.75) (layer F.Cu) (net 15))
 (segment (start 151.86 101.06) (end 151.86 105.41) (width 0.75) (layer F.Cu) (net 15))
 (segment (start 149.86 93.98) (end 149.86 99.06) (width 0.75) (layer F.Cu) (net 15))
 (segment (start 105.41 127) (end 105.41 142.24) (width 0.75) (layer B.Cu) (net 15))
 (segment (start 106.68 125.73) (end 105.41 127) (width 0.75) (layer B.Cu) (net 15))
 (segment (start 116.84 125.73) (end 106.68 125.73) (width 0.75) (layer B.Cu) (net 15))
 (segment (start 123.19 119.38) (end 116.84 125.73) (width 0.75) (layer B.Cu) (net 15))
 (segment (start 137.89 119.38) (end 123.19 119.38) (width 0.75) (layer B.Cu) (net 15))
 (segment (start 151.86 105.41) (end 137.89 119.38) (width 0.75) (layer B.Cu) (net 15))
 (segment (start 160.02 92.71) (end 158.75 91.44) (width 0.75) (layer F.Cu) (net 15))
 (segment (start 149.86 92.71) (end 149.86 93.98) (width 0.75) (layer F.Cu) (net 15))
 (segment (start 151.13 91.44) (end 149.86 92.71) (width 0.75) (layer F.Cu) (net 15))
 (segment (start 158.75 91.44) (end 151.13 91.44) (width 0.75) (layer F.Cu) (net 15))
 (segment (start 156.75 111.76) (end 151.86 111.76) (width 0.75) (layer F.Cu) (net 14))
 (segment (start 152.4 93.98) (end 152.4 97.79) (width 0.75) (layer F.Cu) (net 14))
 (segment (start 156.75 102.14) (end 156.75 111.76) (width 0.75) (layer F.Cu) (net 14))
 (segment (start 152.4 97.79) (end 156.75 102.14) (width 0.75) (layer F.Cu) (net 14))
 (segment (start 130.08 133.35) (end 130.08 136.43) (width 0.75) (layer F.Cu) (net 17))
 (segment (start 137.16 139.7) (end 137.16 142.24) (width 0.75) (layer F.Cu) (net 17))
 (segment (start 135.89 138.43) (end 137.16 139.7) (width 0.75) (layer F.Cu) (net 17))
 (segment (start 132.08 138.43) (end 135.89 138.43) (width 0.75) (layer F.Cu) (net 17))
 (segment (start 130.08 136.43) (end 132.08 138.43) (width 0.75) (layer F.Cu) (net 17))
 (segment (start 134.08 133.35) (end 134.08 134.08) (width 0.75) (layer F.Cu) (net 18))
 (segment (start 134.08 134.08) (end 139.7 139.7) (width 0.75) (layer F.Cu) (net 18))
 (segment (start 139.7 139.7) (end 139.7 142.24) (width 0.75) (layer F.Cu) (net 18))
 (segment (start 134.08 133.35) (end 134.08 133.89) (width 0.75) (layer F.Cu) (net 18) (status 30))
 (segment (start 137.7 133.35) (end 137.7 135.16) (width 0.75) (layer F.Cu) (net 19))
 (segment (start 142.24 139.7) (end 142.24 142.24) (width 0.75) (layer F.Cu) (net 19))
 (segment (start 137.7 135.16) (end 142.24 139.7) (width 0.75) (layer F.Cu) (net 19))
 (segment (start 141.7 133.35) (end 141.7 136.62) (width 0.75) (layer F.Cu) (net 20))
 (segment (start 144.78 139.7) (end 144.78 142.24) (width 0.75) (layer F.Cu) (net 20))
 (segment (start 141.7 136.62) (end 144.78 139.7) (width 0.75) (layer F.Cu) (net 20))
 (segment (start 145.32 133.35) (end 145.32 136.43) (width 0.75) (layer F.Cu) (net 21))
 (segment (start 147.32 138.43) (end 147.32 142.24) (width 0.75) (layer F.Cu) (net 21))
 (segment (start 145.32 136.43) (end 147.32 138.43) (width 0.75) (layer F.Cu) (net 21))
 (segment (start 149.32 133.35) (end 149.32 141.7) (width 0.75) (layer F.Cu) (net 22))
 (segment (start 149.32 141.7) (end 149.86 142.24) (width 0.75) (layer F.Cu) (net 22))
 (segment (start 152.94 133.35) (end 152.94 137.89) (width 0.75) (layer F.Cu) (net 23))
 (segment (start 152.4 138.43) (end 152.4 142.24) (width 0.75) (layer F.Cu) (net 23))
 (segment (start 152.94 137.89) (end 152.4 138.43) (width 0.75) (layer F.Cu) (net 23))
 (segment (start 156.94 133.35) (end 156.94 140.24) (width 0.75) (layer F.Cu) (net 24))
 (segment (start 156.94 140.24) (end 154.94 142.24) (width 0.75) (layer F.Cu) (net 24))
 (segment (start 156.94 133.35) (end 156.94 133.89) (width 0.75) (layer F.Cu) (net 24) (status 30))
 (segment (start 110.49 142.24) (end 110.49 140.97) (width 0.75) (layer F.Cu) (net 26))
 (segment (start 128.27 138.43) (end 132.08 142.24) (width 0.75) (layer F.Cu) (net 26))
 (segment (start 113.03 138.43) (end 128.27 138.43) (width 0.75) (layer F.Cu) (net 26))
 (segment (start 110.49 140.97) (end 113.03 138.43) (width 0.75) (layer F.Cu) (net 26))
 (segment (start 113.03 142.24) (end 113.03 144.78) (width 0.75) (layer F.Cu) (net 25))
 (segment (start 134.62 144.78) (end 134.62 142.24) (width 0.75) (layer F.Cu) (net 25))
 (segment (start 133.35 146.05) (end 134.62 144.78) (width 0.75) (layer F.Cu) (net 25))
 (segment (start 114.3 146.05) (end 133.35 146.05) (width 0.75) (layer F.Cu) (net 25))
 (segment (start 113.03 144.78) (end 114.3 146.05) (width 0.75) (layer F.Cu) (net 25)))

